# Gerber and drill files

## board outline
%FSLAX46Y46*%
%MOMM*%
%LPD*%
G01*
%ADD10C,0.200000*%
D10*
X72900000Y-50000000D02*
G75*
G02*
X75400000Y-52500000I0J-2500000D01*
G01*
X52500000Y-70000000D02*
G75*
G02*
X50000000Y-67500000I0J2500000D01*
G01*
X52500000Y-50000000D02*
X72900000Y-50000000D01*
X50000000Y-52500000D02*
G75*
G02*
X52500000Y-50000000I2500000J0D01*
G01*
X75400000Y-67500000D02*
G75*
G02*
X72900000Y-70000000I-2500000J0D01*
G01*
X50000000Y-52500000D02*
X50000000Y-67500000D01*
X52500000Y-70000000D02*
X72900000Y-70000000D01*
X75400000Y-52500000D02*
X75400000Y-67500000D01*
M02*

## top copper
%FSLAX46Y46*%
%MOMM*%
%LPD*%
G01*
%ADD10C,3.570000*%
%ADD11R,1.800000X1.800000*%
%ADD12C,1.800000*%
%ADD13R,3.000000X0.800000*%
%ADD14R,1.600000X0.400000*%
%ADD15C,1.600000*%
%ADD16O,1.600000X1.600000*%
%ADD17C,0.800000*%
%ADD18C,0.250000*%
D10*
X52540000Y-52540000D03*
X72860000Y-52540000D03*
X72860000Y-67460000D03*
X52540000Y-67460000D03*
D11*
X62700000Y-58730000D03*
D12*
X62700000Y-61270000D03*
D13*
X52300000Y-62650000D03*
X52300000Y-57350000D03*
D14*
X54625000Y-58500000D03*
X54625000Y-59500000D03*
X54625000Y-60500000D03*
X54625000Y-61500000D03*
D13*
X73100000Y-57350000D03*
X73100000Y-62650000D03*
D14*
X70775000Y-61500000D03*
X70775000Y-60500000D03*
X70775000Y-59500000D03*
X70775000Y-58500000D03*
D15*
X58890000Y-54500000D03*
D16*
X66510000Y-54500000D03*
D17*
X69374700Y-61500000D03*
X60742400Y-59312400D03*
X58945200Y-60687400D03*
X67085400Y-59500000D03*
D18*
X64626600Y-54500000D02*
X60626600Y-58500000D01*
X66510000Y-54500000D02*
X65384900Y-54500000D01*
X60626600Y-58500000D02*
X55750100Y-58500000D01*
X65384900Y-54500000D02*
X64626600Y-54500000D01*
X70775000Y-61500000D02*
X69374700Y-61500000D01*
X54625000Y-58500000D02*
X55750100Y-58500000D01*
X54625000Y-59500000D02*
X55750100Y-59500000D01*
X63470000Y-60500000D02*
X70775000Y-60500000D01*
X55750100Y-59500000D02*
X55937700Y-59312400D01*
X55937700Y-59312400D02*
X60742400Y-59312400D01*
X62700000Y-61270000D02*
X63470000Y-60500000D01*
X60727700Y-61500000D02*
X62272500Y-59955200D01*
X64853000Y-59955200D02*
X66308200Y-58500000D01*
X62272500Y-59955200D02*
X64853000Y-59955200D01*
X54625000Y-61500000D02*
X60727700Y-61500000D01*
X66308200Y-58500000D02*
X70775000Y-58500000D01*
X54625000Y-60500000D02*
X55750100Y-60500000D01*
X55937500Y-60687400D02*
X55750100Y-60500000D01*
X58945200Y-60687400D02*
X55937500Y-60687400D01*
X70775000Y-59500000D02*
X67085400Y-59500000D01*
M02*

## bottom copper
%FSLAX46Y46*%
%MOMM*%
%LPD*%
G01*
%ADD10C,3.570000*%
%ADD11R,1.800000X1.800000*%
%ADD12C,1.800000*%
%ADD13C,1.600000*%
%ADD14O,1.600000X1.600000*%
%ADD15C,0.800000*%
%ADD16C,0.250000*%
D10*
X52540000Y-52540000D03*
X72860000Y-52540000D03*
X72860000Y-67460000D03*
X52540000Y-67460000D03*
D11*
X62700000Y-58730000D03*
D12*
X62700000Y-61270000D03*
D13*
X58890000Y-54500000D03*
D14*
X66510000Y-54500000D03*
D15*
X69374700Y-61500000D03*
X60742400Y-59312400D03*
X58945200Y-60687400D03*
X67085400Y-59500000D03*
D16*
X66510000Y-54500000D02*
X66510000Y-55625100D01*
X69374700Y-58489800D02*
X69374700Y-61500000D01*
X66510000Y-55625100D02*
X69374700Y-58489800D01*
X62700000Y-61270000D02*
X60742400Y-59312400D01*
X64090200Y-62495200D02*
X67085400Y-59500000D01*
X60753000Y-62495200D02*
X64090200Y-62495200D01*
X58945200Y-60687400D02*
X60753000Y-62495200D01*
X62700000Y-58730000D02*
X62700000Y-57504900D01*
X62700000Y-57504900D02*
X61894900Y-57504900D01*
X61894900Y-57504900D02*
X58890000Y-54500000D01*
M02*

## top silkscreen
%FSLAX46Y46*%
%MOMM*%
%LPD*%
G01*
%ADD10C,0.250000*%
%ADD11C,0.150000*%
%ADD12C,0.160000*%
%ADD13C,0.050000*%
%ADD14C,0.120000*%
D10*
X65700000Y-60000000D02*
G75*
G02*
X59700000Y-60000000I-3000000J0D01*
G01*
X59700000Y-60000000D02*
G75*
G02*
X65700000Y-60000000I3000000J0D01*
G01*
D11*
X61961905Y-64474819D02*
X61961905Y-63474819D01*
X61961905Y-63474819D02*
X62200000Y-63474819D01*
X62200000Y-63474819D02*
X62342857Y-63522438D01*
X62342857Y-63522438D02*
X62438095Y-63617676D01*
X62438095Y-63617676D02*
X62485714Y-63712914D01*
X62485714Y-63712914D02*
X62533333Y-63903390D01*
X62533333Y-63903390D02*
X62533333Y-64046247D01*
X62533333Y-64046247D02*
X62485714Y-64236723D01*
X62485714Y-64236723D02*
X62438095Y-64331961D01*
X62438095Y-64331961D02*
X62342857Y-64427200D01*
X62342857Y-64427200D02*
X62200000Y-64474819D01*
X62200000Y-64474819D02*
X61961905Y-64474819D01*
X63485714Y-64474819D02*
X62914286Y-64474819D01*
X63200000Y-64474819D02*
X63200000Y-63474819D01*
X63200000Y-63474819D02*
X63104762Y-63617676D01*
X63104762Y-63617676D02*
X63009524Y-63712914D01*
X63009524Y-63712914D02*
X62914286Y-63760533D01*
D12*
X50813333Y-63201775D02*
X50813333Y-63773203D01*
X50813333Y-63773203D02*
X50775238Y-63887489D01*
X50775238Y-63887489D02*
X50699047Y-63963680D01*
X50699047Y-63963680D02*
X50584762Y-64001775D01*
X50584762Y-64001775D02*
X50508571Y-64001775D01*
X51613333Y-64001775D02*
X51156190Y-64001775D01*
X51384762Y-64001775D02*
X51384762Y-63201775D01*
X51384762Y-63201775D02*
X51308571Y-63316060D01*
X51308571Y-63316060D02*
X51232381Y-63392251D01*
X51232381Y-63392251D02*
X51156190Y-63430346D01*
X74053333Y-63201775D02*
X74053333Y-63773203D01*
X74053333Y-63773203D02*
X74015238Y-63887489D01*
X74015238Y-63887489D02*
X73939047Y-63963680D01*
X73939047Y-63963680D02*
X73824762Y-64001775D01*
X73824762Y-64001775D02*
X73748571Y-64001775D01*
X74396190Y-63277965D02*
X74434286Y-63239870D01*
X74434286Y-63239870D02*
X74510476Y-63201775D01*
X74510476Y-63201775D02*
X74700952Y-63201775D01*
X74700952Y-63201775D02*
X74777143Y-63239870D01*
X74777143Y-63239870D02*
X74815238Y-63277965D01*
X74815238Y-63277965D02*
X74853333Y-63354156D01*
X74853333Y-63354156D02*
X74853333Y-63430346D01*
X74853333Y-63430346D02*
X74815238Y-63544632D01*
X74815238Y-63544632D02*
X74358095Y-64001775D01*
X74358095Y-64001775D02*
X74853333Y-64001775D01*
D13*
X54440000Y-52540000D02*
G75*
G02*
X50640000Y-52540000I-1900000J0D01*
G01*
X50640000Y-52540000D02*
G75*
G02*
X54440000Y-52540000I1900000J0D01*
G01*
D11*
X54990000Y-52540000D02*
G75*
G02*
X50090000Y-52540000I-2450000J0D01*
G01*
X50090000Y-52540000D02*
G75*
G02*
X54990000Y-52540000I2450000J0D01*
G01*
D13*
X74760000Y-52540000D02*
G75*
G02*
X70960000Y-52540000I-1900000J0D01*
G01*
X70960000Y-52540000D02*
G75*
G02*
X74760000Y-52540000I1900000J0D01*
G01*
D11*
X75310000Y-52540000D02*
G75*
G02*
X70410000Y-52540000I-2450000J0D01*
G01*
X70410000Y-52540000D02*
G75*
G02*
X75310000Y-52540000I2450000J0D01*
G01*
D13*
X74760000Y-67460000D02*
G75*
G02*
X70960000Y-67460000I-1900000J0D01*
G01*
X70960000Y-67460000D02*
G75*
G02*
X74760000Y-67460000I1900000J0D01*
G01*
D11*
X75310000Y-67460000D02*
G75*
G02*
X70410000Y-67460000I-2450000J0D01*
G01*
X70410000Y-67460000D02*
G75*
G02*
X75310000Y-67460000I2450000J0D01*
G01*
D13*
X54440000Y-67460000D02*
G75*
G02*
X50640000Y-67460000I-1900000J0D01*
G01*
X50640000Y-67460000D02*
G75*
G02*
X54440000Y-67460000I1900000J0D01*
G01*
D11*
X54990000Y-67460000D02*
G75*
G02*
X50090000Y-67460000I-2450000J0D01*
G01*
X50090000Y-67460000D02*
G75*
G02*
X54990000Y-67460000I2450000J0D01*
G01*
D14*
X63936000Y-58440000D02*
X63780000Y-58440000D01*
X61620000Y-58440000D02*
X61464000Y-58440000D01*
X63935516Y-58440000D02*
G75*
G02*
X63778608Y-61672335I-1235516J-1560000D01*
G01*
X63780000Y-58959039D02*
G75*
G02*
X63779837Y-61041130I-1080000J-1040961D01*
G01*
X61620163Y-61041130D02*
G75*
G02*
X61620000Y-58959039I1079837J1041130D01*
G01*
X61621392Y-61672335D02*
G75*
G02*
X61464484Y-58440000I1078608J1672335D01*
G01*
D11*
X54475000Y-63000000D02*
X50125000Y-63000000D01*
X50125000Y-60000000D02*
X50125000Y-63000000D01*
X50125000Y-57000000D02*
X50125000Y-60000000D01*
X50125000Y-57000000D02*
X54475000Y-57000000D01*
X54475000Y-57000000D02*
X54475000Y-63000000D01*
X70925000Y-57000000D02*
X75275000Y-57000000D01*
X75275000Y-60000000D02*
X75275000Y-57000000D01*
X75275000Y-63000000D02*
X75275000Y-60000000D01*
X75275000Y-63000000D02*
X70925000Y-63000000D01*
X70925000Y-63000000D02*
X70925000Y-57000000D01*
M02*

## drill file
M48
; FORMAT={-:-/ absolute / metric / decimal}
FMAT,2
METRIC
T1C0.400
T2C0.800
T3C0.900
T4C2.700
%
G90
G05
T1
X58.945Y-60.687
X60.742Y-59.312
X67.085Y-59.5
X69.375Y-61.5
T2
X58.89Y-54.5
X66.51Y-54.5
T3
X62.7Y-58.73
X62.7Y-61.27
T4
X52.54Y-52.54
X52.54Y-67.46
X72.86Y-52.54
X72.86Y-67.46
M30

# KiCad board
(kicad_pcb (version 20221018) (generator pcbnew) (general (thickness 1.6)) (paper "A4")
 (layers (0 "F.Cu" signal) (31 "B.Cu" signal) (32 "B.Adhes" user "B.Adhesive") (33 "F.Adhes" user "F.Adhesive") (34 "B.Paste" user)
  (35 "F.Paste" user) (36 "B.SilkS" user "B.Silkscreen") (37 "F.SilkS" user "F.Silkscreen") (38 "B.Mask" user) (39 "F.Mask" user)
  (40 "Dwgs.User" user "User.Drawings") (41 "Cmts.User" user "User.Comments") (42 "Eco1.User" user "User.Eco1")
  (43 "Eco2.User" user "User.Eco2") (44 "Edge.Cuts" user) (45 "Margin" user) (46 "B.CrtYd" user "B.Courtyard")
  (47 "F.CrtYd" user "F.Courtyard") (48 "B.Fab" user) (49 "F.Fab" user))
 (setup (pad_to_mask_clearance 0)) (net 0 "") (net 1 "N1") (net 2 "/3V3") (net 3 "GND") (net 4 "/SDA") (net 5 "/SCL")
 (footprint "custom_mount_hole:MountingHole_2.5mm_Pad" (layer "F.Cu") (at 52.54 52.54)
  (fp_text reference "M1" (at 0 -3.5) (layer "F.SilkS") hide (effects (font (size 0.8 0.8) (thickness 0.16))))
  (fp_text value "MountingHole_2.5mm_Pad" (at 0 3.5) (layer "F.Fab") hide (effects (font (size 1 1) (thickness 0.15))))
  (fp_circle (center 0 0) (end 1.9 0) (stroke (width 0.05) (type solid)) (fill none) (layer "F.SilkS"))
  (fp_circle (center 0 0) (end 2.45 0) (stroke (width 0.15) (type solid)) (fill none) (layer "F.SilkS"))
  (pad "~" thru_hole circle (at 0 0) (size 3.57 3.57) (drill 2.7) (layers "*.Cu" "*.Mask")))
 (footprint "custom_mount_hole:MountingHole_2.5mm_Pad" (layer "F.Cu") (at 72.86 52.54)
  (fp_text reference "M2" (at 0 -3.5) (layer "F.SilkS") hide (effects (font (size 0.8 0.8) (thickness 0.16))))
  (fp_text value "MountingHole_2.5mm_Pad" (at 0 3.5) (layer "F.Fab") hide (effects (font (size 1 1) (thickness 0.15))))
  (fp_circle (center 0 0) (end 1.9 0) (stroke (width 0.05) (type solid)) (fill none) (layer "F.SilkS"))
  (fp_circle (center 0 0) (end 2.45 0) (stroke (width 0.15) (type solid)) (fill none) (layer "F.SilkS"))
  (pad "~" thru_hole circle (at 0 0) (size 3.57 3.57) (drill 2.7) (layers "*.Cu" "*.Mask")))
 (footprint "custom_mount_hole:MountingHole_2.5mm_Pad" (layer "F.Cu") (at 72.86 67.46)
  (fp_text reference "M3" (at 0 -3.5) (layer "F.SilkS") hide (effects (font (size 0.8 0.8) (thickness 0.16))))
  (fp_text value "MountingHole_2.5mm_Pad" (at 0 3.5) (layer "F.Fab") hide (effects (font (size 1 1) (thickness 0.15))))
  (fp_circle (center 0 0) (end 1.9 0) (stroke (width 0.05) (type solid)) (fill none) (layer "F.SilkS"))
  (fp_circle (center 0 0) (end 2.45 0) (stroke (width 0.15) (type solid)) (fill none) (layer "F.SilkS"))
  (pad "~" thru_hole circle (at 0 0) (size 3.57 3.57) (drill 2.7) (layers "*.Cu" "*.Mask")))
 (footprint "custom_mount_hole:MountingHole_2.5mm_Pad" (layer "F.Cu") (at 52.54 67.46)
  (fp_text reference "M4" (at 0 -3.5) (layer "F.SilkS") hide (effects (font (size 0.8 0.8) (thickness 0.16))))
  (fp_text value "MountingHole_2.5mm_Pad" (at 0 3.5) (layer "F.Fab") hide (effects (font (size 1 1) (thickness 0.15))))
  (fp_circle (center 0 0) (end 1.9 0) (stroke (width 0.05) (type solid)) (fill none) (layer "F.SilkS"))
  (fp_circle (center 0 0) (end 2.45 0) (stroke (width 0.15) (type solid)) (fill none) (layer "F.SilkS"))
  (pad "~" thru_hole circle (at 0 0) (size 3.57 3.57) (drill 2.7) (layers "*.Cu" "*.Mask")))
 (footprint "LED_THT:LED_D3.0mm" (layer "F.Cu") (at 62.7 58.73 -90)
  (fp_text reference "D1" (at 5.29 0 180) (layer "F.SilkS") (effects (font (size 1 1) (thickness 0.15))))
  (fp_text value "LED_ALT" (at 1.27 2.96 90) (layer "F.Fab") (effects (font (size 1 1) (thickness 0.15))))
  (fp_line (start -0.29 -1.236) (end -0.29 -1.08) (stroke (width 0.12) (type solid)) (layer "F.SilkS"))
  (fp_line (start -0.29 1.08) (end -0.29 1.236) (stroke (width 0.12) (type solid)) (layer "F.SilkS"))
  (fp_arc (start -0.29 -1.235516) (mid 1.366487 -1.987659) (end 2.942335 -1.078608) (stroke (width 0.12) (type solid)) (layer "F.SilkS"))
  (fp_arc (start 0.229039 -1.08) (mid 1.270117 -1.5) (end 2.31113 -1.079837) (stroke (width 0.12) (type solid)) (layer "F.SilkS"))
  (fp_arc (start 2.31113 1.079837) (mid 1.270117 1.5) (end 0.229039 1.08) (stroke (width 0.12) (type solid)) (layer "F.SilkS"))
  (fp_arc (start 2.942335 1.078608) (mid 1.366487 1.987659) (end -0.29 1.235516) (stroke (width 0.12) (type solid)) (layer "F.SilkS"))
  (pad "1" thru_hole rect (at 0 0 270) (size 1.8 1.8) (drill 0.9) (layers "*.Cu" "*.Mask") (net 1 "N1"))
  (pad "2" thru_hole circle (at 2.54 0 270) (size 1.8 1.8) (drill 0.9) (layers "*.Cu" "*.Mask") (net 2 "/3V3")))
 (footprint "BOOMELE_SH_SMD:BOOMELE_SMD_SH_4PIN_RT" (layer "F.Cu") (at 52.78 60 90)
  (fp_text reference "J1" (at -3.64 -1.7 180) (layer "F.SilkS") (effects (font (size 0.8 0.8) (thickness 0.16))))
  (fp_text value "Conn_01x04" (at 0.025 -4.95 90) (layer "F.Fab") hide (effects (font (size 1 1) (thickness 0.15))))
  (fp_line (start -3 1.695) (end -3 -2.655) (stroke (width 0.15) (type solid)) (layer "F.SilkS"))
  (fp_line (start 0 -2.655) (end -3 -2.655) (stroke (width 0.15) (type solid)) (layer "F.SilkS"))
  (fp_line (start 3 -2.655) (end 0 -2.655) (stroke (width 0.15) (type solid)) (layer "F.SilkS"))
  (fp_line (start 3 -2.655) (end 3 1.695) (stroke (width 0.15) (type solid)) (layer "F.SilkS"))
  (fp_line (start 3 1.695) (end -3 1.695) (stroke (width 0.15) (type solid)) (layer "F.SilkS"))
  (pad "" smd rect (at -2.65 -0.48 270) (size 0.8 3) (layers "F.Cu" "F.Paste" "F.Mask"))
  (pad "" smd rect (at 2.65 -0.48 270) (size 0.8 3) (layers "F.Cu" "F.Paste" "F.Mask"))
  (pad "1" smd rect (at 1.5 1.845 270) (size 0.4 1.6) (layers "F.Cu" "F.Paste" "F.Mask") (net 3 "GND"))
  (pad "2" smd rect (at 0.5 1.845 270) (size 0.4 1.6) (layers "F.Cu" "F.Paste" "F.Mask") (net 2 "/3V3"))
  (pad "3" smd rect (at -0.5 1.845 270) (size 0.4 1.6) (layers "F.Cu" "F.Paste" "F.Mask") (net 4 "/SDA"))
  (pad "4" smd rect (at -1.5 1.845 270) (size 0.4 1.6) (layers "F.Cu" "F.Paste" "F.Mask") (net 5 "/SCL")))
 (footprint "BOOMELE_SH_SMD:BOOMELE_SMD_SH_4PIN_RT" (layer "F.Cu") (at 72.62 60 -90)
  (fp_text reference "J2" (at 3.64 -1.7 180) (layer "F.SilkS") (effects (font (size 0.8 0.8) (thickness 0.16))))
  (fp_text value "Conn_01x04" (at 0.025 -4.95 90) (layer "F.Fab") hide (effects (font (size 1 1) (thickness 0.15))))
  (fp_line (start -3 1.695) (end -3 -2.655) (stroke (width 0.15) (type solid)) (layer "F.SilkS"))
  (fp_line (start 0 -2.655) (end -3 -2.655) (stroke (width 0.15) (type solid)) (layer "F.SilkS"))
  (fp_line (start 3 -2.655) (end 0 -2.655) (stroke (width 0.15) (type solid)) (layer "F.SilkS"))
  (fp_line (start 3 -2.655) (end 3 1.695) (stroke (width 0.15) (type solid)) (layer "F.SilkS"))
  (fp_line (start 3 1.695) (end -3 1.695) (stroke (width 0.15) (type solid)) (layer "F.SilkS"))
  (pad "" smd rect (at -2.65 -0.48 90) (size 0.8 3) (layers "F.Cu" "F.Paste" "F.Mask"))
  (pad "" smd rect (at 2.65 -0.48 90) (size 0.8 3) (layers "F.Cu" "F.Paste" "F.Mask"))
  (pad "1" smd rect (at 1.5 1.845 90) (size 0.4 1.6) (layers "F.Cu" "F.Paste" "F.Mask") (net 3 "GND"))
  (pad "2" smd rect (at 0.5 1.845 90) (size 0.4 1.6) (layers "F.Cu" "F.Paste" "F.Mask") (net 2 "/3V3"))
  (pad "3" smd rect (at -0.5 1.845 90) (size 0.4 1.6) (layers "F.Cu" "F.Paste" "F.Mask") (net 4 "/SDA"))
  (pad "4" smd rect (at -1.5 1.845 90) (size 0.4 1.6) (layers "F.Cu" "F.Paste" "F.Mask") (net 5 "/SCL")))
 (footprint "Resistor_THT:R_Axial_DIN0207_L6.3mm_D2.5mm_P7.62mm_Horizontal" (layer "B.Cu") (at 58.89 54.5)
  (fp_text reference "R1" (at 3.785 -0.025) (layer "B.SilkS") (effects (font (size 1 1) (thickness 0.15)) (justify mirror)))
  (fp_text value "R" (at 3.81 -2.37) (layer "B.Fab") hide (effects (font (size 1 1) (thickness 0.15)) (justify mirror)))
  (pad "1" thru_hole circle (at 0 0) (size 1.6 1.6) (drill 0.8) (layers "*.Cu" "*.Mask") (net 1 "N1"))
  (pad "2" thru_hole oval (at 7.62 0) (size 1.6 1.6) (drill 0.8) (layers "*.Cu" "*.Mask") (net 3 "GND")))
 (gr_circle (center 62.7 60) (end 65.7 60) (stroke (width 0.25) (type solid)) (fill none) (layer "F.SilkS"))
 (gr_arc (start 72.9 50) (mid 74.667767 50.732233) (end 75.4 52.5) (stroke (width 0.2) (type solid)) (layer "Edge.Cuts"))
 (gr_arc (start 52.5 70) (mid 50.732233 69.267767) (end 50 67.5) (stroke (width 0.2) (type solid)) (layer "Edge.Cuts"))
 (gr_line (start 52.5 50) (end 72.9 50) (stroke (width 0.2) (type solid)) (layer "Edge.Cuts"))
 (gr_arc (start 50 52.5) (mid 50.732233 50.732233) (end 52.5 50) (stroke (width 0.2) (type solid)) (layer "Edge.Cuts"))
 (gr_arc (start 75.4 67.5) (mid 74.667767 69.267767) (end 72.9 70) (stroke (width 0.2) (type solid)) (layer "Edge.Cuts"))
 (gr_line (start 50 52.5) (end 50 67.5) (stroke (width 0.2) (type solid)) (layer "Edge.Cuts"))
 (gr_line (start 52.5 70) (end 72.9 70) (stroke (width 0.2) (type solid)) (layer "Edge.Cuts"))
 (gr_line (start 75.4 52.5) (end 75.4 67.5) (stroke (width 0.2) (type solid)) (layer "Edge.Cuts"))
 (segment (start 64.6266 54.5) (end 60.6266 58.5) (width 0.25) (layer "F.Cu") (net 3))
 (segment (start 66.51 54.5) (end 65.3849 54.5) (width 0.25) (layer "F.Cu") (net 3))
 (segment (start 60.6266 58.5) (end 55.7501 58.5) (width 0.25) (layer "F.Cu") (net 3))
 (segment (start 65.3849 54.5) (end 64.6266 54.5) (width 0.25) (layer "F.Cu") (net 3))
 (segment (start 70.775 61.5) (end 69.3747 61.5) (width 0.25) (layer "F.Cu") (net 3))
 (segment (start 54.625 58.5) (end 55.7501 58.5) (width 0.25) (layer "F.Cu") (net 3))
 (via (at 69.3747 61.5) (size 0.8) (drill 0.4) (layers "F.Cu" "B.Cu") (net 3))
 (segment (start 66.51 54.5) (end 66.51 55.6251) (width 0.25) (layer "B.Cu") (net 3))
 (segment (start 69.3747 58.4898) (end 69.3747 61.5) (width 0.25) (layer "B.Cu") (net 3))
 (segment (start 66.51 55.6251) (end 69.3747 58.4898) (width 0.25) (layer "B.Cu") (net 3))
 (segment (start 54.625 59.5) (end 55.7501 59.5) (width 0.25) (layer "F.Cu") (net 2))
 (segment (start 63.47 60.5) (end 70.775 60.5) (width 0.25) (layer "F.Cu") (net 2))
 (segment (start 55.7501 59.5) (end 55.9377 59.3124) (width 0.25) (layer "F.Cu") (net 2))
 (segment (start 55.9377 59.3124) (end 60.7424 59.3124) (width 0.25) (layer "F.Cu") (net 2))
 (segment (start 62.7 61.27) (end 63.47 60.5) (width 0.25) (layer "F.Cu") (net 2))
 (via (at 60.7424 59.3124) (size 0.8) (drill 0.4) (layers "F.Cu" "B.Cu") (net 2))
 (segment (start 62.7 61.27) (end 60.7424 59.3124) (width 0.25) (layer "B.Cu") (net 2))
 (segment (start 60.7277 61.5) (end 62.2725 59.9552) (width 0.25) (layer "F.Cu") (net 5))
 (segment (start 64.853 59.9552) (end 66.3082 58.5) (width 0.25) (layer "F.Cu") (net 5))
 (segment (start 62.2725 59.9552) (end 64.853 59.9552) (width 0.25) (layer "F.Cu") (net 5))
 (segment (start 54.625 61.5) (end 60.7277 61.5) (width 0.25) (layer "F.Cu") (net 5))
 (segment (start 66.3082 58.5) (end 70.775 58.5) (width 0.25) (layer "F.Cu") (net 5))
 (segment (start 54.625 60.5) (end 55.7501 60.5) (width 0.25) (layer "F.Cu") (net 4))
 (segment (start 55.9375 60.6874) (end 55.7501 60.5) (width 0.25) (layer "F.Cu") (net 4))
 (segment (start 58.9452 60.6874) (end 55.9375 60.6874) (width 0.25) (layer "F.Cu") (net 4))
 (segment (start 70.775 59.5) (end 67.0854 59.5) (width 0.25) (layer "F.Cu") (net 4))
 (via (at 58.9452 60.6874) (size 0.8) (drill 0.4) (layers "F.Cu" "B.Cu") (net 4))
 (via (at 67.0854 59.5) (size 0.8) (drill 0.4) (layers "F.Cu" "B.Cu") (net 4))
 (segment (start 64.0902 62.4952) (end 67.0854 59.5) (width 0.25) (layer "B.Cu") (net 4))
 (segment (start 60.753 62.4952) (end 64.0902 62.4952) (width 0.25) (layer "B.Cu") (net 4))
 (segment (start 58.9452 60.6874) (end 60.753 62.4952) (width 0.25) (layer "B.Cu") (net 4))
 (segment (start 62.7 58.73) (end 62.7 57.5049) (width 0.25) (layer "B.Cu") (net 1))
 (segment (start 62.7 57.5049) (end 61.8949 57.5049) (width 0.25) (layer "B.Cu") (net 1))
 (segment (start 61.8949 57.5049) (end 58.89 54.5) (width 0.25) (layer "B.Cu") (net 1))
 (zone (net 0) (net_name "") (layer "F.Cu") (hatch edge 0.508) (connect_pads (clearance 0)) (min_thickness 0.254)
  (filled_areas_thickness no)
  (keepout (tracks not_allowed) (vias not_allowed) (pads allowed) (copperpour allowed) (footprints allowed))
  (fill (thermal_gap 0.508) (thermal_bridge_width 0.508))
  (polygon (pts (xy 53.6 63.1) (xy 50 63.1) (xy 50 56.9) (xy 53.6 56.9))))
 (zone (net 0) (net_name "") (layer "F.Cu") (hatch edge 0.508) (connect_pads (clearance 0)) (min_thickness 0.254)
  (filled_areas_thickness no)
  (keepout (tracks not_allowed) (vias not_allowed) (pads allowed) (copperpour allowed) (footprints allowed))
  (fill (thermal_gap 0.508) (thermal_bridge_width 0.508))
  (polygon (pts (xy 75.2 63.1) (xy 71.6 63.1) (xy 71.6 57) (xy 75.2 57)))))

